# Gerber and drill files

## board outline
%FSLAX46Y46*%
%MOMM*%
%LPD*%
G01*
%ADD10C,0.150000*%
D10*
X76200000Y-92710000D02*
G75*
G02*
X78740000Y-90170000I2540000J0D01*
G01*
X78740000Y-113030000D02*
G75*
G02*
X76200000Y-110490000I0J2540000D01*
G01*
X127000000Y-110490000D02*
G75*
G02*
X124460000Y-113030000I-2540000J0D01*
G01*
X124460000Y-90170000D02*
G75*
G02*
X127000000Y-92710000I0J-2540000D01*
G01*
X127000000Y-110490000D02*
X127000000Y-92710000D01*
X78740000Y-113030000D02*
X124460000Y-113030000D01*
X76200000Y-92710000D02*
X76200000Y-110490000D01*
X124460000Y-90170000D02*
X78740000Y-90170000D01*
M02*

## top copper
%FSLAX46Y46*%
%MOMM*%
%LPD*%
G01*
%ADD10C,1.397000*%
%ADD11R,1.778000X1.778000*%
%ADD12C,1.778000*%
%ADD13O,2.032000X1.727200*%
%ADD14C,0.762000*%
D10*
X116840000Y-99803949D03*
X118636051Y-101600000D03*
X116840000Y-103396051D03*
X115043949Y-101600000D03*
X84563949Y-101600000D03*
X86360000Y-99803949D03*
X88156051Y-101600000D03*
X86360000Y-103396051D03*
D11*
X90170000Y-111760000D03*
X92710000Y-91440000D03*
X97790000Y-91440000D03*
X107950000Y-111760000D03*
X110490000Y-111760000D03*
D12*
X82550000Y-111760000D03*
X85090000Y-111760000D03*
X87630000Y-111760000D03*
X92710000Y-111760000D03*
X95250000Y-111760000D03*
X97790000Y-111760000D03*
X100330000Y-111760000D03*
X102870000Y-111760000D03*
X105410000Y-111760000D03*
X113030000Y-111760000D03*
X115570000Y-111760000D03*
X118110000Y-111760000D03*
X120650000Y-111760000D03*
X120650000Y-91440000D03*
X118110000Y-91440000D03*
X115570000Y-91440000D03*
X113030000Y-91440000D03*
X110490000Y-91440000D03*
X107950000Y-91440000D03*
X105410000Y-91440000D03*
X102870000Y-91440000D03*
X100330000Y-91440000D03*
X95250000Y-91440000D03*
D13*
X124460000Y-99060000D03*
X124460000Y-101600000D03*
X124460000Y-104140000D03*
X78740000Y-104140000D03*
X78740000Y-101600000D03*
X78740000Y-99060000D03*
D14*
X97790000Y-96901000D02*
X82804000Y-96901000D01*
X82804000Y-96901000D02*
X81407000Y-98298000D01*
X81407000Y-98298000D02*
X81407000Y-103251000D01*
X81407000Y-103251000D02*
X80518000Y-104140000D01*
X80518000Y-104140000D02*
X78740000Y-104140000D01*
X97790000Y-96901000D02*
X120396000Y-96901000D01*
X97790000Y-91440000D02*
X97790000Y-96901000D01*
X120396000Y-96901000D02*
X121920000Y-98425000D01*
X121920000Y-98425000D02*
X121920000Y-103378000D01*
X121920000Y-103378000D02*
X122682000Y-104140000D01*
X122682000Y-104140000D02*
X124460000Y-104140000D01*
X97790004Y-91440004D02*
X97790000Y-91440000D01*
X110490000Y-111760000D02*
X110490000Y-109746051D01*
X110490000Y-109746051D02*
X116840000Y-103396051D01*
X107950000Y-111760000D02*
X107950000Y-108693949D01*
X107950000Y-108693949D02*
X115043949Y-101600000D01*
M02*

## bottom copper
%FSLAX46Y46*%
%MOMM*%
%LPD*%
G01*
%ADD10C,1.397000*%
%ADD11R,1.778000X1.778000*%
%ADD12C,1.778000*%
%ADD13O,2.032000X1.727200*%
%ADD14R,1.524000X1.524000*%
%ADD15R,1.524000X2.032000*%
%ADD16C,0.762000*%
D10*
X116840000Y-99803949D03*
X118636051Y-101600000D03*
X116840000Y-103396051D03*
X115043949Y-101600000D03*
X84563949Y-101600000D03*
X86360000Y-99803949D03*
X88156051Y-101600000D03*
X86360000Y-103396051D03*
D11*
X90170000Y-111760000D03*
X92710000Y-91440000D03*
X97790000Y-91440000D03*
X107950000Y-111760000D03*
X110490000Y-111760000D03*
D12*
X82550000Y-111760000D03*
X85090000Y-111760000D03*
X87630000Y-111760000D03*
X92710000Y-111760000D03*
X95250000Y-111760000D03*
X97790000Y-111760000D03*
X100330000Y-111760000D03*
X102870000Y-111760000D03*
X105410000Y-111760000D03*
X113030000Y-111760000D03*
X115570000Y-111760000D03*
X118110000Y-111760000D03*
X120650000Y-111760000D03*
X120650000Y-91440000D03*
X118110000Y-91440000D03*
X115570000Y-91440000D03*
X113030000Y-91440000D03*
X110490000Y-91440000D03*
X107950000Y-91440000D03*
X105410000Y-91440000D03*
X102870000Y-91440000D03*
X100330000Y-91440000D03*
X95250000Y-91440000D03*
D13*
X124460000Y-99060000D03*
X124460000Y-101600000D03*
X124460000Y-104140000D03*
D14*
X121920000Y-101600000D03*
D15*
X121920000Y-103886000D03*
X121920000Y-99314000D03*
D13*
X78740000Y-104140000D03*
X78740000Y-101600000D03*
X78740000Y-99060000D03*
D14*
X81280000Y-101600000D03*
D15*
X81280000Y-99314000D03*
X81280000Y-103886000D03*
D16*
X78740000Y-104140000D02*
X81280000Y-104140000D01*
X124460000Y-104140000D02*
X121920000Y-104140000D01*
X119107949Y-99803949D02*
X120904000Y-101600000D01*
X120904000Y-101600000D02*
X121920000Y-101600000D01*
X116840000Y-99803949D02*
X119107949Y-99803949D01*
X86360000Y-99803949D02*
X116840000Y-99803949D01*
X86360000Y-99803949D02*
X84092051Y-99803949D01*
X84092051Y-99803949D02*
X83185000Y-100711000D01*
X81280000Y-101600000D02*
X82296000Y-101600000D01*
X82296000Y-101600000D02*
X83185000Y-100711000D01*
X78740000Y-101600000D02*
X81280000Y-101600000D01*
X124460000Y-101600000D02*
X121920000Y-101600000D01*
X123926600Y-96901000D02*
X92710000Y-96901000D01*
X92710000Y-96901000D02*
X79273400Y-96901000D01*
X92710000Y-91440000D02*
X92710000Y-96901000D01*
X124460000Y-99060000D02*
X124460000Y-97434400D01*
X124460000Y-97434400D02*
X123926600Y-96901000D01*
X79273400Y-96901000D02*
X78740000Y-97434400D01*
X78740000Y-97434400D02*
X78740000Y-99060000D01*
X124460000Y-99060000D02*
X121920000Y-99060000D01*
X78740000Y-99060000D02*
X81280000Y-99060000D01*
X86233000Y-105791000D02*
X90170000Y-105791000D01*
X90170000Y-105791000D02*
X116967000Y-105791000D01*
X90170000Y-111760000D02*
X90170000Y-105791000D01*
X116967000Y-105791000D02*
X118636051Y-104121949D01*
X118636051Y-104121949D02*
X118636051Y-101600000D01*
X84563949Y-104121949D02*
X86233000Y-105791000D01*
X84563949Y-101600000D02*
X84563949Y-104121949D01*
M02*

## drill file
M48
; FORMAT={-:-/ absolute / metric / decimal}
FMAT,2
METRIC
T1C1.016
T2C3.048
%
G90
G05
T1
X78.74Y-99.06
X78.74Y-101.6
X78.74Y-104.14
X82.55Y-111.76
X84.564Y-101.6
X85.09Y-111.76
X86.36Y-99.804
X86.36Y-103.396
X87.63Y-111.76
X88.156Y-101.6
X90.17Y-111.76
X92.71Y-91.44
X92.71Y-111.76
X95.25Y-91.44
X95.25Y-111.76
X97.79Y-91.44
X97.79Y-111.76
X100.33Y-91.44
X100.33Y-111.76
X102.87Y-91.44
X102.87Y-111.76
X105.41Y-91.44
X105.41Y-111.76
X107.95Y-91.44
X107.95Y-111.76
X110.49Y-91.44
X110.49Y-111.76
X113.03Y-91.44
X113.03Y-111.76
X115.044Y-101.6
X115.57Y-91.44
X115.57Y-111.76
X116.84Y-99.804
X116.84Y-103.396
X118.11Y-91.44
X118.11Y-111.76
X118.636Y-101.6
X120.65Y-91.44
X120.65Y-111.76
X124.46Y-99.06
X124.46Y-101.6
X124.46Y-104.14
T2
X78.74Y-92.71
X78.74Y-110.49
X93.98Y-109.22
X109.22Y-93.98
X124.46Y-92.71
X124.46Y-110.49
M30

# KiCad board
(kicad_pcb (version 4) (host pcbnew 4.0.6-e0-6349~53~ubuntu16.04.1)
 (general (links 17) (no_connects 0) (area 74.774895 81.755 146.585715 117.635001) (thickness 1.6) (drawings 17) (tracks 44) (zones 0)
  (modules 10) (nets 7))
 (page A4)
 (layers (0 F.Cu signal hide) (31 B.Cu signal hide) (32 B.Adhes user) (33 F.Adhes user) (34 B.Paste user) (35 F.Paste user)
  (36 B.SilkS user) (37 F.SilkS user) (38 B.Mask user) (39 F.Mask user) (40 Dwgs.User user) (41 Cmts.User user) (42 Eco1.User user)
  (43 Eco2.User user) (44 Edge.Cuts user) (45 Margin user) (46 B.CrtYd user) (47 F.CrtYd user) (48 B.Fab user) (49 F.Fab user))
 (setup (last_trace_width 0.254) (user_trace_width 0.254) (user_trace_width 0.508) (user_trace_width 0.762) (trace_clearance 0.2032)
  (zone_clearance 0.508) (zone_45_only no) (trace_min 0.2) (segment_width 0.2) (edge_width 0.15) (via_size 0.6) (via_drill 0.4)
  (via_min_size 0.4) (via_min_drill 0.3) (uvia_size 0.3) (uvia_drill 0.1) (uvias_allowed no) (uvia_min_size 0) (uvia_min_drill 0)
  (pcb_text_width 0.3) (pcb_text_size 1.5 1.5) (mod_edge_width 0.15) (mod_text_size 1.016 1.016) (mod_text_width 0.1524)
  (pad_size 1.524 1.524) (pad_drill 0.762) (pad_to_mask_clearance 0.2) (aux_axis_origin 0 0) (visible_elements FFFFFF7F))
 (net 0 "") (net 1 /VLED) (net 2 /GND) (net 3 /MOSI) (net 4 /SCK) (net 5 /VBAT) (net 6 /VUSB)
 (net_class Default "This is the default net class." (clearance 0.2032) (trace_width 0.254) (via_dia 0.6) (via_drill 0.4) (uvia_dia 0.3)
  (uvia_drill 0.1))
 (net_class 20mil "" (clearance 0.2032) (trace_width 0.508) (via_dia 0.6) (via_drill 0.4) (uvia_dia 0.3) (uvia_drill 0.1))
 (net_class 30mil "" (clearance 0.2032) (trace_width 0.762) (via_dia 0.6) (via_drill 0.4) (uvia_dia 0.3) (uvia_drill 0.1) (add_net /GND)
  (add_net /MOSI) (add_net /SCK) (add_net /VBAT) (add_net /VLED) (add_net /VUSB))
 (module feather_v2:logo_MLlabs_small (layer F.Cu) (at 107.95 101.6 90)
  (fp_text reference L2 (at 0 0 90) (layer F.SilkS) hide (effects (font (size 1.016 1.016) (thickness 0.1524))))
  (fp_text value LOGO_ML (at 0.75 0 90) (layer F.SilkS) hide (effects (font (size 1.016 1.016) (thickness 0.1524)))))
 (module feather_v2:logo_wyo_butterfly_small (layer F.Cu) (at 99.187 101.6 45)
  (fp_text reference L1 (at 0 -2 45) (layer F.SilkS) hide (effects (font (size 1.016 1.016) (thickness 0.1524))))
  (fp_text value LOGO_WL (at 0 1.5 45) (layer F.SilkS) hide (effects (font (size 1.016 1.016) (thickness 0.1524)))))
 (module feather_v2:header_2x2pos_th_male (layer B.Cu) (at 116.84 101.6 315)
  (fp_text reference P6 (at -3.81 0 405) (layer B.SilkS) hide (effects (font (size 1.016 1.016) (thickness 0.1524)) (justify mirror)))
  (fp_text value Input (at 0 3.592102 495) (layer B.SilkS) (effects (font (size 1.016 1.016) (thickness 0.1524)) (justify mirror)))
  (pad 1 thru_hole circle (at -1.27 -1.27 315) (size 1.397 1.397) (drill 1.016) (layers *.Cu *.Mask B.SilkS) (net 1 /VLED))
  (pad 3 thru_hole circle (at 1.27 -1.27 315) (size 1.397 1.397) (drill 1.016) (layers *.Cu *.Mask B.SilkS) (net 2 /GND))
  (pad 4 thru_hole circle (at 1.27 1.27 315) (size 1.397 1.397) (drill 1.016) (layers *.Cu *.Mask B.SilkS) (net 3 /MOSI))
  (pad 2 thru_hole circle (at -1.27 1.27 315) (size 1.397 1.397) (drill 1.016) (layers *.Cu *.Mask B.SilkS) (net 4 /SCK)))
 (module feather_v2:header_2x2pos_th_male (layer B.Cu) (at 86.36 101.6 45)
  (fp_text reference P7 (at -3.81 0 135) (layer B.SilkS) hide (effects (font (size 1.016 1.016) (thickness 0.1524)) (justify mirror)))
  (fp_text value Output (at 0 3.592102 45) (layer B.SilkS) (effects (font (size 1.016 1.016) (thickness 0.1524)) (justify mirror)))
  (pad 1 thru_hole circle (at -1.27 -1.27 45) (size 1.397 1.397) (drill 1.016) (layers *.Cu *.Mask B.SilkS) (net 2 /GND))
  (pad 3 thru_hole circle (at 1.27 -1.27 45) (size 1.397 1.397) (drill 1.016) (layers *.Cu *.Mask B.SilkS) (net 1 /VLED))
  (pad 4 thru_hole circle (at 1.27 1.27 45) (size 1.397 1.397) (drill 1.016) (layers *.Cu *.Mask B.SilkS))
  (pad 2 thru_hole circle (at -1.27 1.27 45) (size 1.397 1.397) (drill 1.016) (layers *.Cu *.Mask B.SilkS)))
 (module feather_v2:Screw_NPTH (layer F.Cu) (at 109.22 93.98)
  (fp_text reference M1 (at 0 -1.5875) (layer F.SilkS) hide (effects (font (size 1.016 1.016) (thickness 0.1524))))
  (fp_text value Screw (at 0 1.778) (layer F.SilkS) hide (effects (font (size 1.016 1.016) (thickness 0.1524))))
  (pad "" np_thru_hole circle (at 0 0) (size 3.048 3.048) (drill 3.048) (layers *.Cu *.Mask F.SilkS)))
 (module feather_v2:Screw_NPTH (layer F.Cu) (at 93.98 109.22)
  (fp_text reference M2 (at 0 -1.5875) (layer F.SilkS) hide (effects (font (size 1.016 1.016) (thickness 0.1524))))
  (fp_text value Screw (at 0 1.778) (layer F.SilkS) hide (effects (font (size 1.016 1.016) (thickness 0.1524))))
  (pad "" np_thru_hole circle (at 0 0) (size 3.048 3.048) (drill 3.048) (layers *.Cu *.Mask F.SilkS)))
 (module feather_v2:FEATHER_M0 (layer F.Cu) (at 101.6 101.6)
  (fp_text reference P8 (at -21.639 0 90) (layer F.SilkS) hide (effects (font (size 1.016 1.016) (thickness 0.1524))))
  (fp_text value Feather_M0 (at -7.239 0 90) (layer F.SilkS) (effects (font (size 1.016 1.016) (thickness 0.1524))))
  (pad 4 thru_hole rect (at -11.43 10.16) (size 1.778 1.778) (drill 1.016) (layers *.Cu *.Mask) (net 2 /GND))
  (pad 28 thru_hole rect (at -8.89 -10.16) (size 1.778 1.778) (drill 1.016) (layers *.Cu *.Mask) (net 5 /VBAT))
  (pad 26 thru_hole rect (at -3.81 -10.16) (size 1.778 1.778) (drill 1.016) (layers *.Cu *.Mask) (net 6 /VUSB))
  (pad 11 thru_hole rect (at 6.35 10.16) (size 1.778 1.778) (drill 1.016) (layers *.Cu *.Mask) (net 4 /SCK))
  (pad 12 thru_hole rect (at 8.89 10.16) (size 1.778 1.778) (drill 1.016) (layers *.Cu *.Mask) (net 3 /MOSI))
  (pad 1 thru_hole circle (at -19.05 10.16) (size 1.778 1.778) (drill 1.016) (layers *.Cu *.Mask))
  (pad 2 thru_hole circle (at -16.51 10.16) (size 1.778 1.778) (drill 1.016) (layers *.Cu *.Mask))
  (pad 3 thru_hole circle (at -13.97 10.16) (size 1.778 1.778) (drill 1.016) (layers *.Cu *.Mask))
  (pad 5 thru_hole circle (at -8.89 10.16) (size 1.778 1.778) (drill 1.016) (layers *.Cu *.Mask))
  (pad 6 thru_hole circle (at -6.35 10.16) (size 1.778 1.778) (drill 1.016) (layers *.Cu *.Mask))
  (pad 7 thru_hole circle (at -3.81 10.16) (size 1.778 1.778) (drill 1.016) (layers *.Cu *.Mask))
  (pad 8 thru_hole circle (at -1.27 10.16) (size 1.778 1.778) (drill 1.016) (layers *.Cu *.Mask))
  (pad 9 thru_hole circle (at 1.27 10.16) (size 1.778 1.778) (drill 1.016) (layers *.Cu *.Mask))
  (pad 10 thru_hole circle (at 3.81 10.16) (size 1.778 1.778) (drill 1.016) (layers *.Cu *.Mask))
  (pad 13 thru_hole circle (at 11.43 10.16) (size 1.778 1.778) (drill 1.016) (layers *.Cu *.Mask))
  (pad 14 thru_hole circle (at 13.97 10.16) (size 1.778 1.778) (drill 1.016) (layers *.Cu *.Mask))
  (pad 15 thru_hole circle (at 16.51 10.16) (size 1.778 1.778) (drill 1.016) (layers *.Cu *.Mask))
  (pad 16 thru_hole circle (at 19.05 10.16) (size 1.778 1.778) (drill 1.016) (layers *.Cu *.Mask))
  (pad 17 thru_hole circle (at 19.05 -10.16) (size 1.778 1.778) (drill 1.016) (layers *.Cu *.Mask))
  (pad 18 thru_hole circle (at 16.51 -10.16) (size 1.778 1.778) (drill 1.016) (layers *.Cu *.Mask))
  (pad 19 thru_hole circle (at 13.97 -10.16) (size 1.778 1.778) (drill 1.016) (layers *.Cu *.Mask))
  (pad 20 thru_hole circle (at 11.43 -10.16) (size 1.778 1.778) (drill 1.016) (layers *.Cu *.Mask))
  (pad 21 thru_hole circle (at 8.89 -10.16) (size 1.778 1.778) (drill 1.016) (layers *.Cu *.Mask))
  (pad 22 thru_hole circle (at 6.35 -10.16) (size 1.778 1.778) (drill 1.016) (layers *.Cu *.Mask))
  (pad 23 thru_hole circle (at 3.81 -10.16) (size 1.778 1.778) (drill 1.016) (layers *.Cu *.Mask))
  (pad 24 thru_hole circle (at 1.27 -10.16) (size 1.778 1.778) (drill 1.016) (layers *.Cu *.Mask))
  (pad 25 thru_hole circle (at -1.27 -10.16) (size 1.778 1.778) (drill 1.016) (layers *.Cu *.Mask))
  (pad 27 thru_hole circle (at -6.35 -10.16) (size 1.778 1.778) (drill 1.016) (layers *.Cu *.Mask))
  (pad "" np_thru_hole circle (at -22.86 8.89) (size 3.048 3.048) (drill 3.048) (layers *.Cu *.Mask))
  (pad "" np_thru_hole circle (at 22.86 8.89) (size 3.048 3.048) (drill 3.048) (layers *.Cu *.Mask))
  (pad "" np_thru_hole circle (at 22.86 -8.89) (size 3.048 3.048) (drill 3.048) (layers *.Cu *.Mask))
  (pad "" np_thru_hole circle (at -22.86 -8.89) (size 3.048 3.048) (drill 3.048) (layers *.Cu *.Mask)))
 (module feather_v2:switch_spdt (layer B.Cu) (at 124.46 101.6 180)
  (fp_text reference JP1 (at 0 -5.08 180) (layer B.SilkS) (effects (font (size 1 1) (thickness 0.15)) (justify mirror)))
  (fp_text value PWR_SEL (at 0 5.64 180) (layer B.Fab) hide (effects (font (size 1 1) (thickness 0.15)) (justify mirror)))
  (pad 1 thru_hole oval (at 0 2.54 180) (size 2.032 1.7272) (drill 1.016) (layers *.Cu *.Mask B.SilkS) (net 5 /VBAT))
  (pad 2 thru_hole oval (at 0 0 180) (size 2.032 1.7272) (drill 1.016) (layers *.Cu *.Mask B.SilkS) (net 1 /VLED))
  (pad 3 thru_hole oval (at 0 -2.54 180) (size 2.032 1.7272) (drill 1.016) (layers *.Cu *.Mask B.SilkS) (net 6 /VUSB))
  (pad 2 smd rect (at 2.54 0 180) (size 1.524 1.524) (layers B.Cu B.Paste B.Mask) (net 1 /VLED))
  (pad 3 smd rect (at 2.54 -2.54 180) (size 1.524 2.032) (drill (offset 0 0.254)) (layers B.Cu B.Paste B.Mask) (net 6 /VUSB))
  (pad 1 smd rect (at 2.54 2.54 180) (size 1.524 2.032) (drill (offset 0 -0.254)) (layers B.Cu B.Paste B.Mask) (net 5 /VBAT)))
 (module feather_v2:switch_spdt (layer B.Cu) (at 78.74 101.6)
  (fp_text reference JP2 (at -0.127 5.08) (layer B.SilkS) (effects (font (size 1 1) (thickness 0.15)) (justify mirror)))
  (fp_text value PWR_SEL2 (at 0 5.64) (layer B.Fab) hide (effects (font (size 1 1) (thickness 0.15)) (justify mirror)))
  (pad 1 thru_hole oval (at 0 2.54) (size 2.032 1.7272) (drill 1.016) (layers *.Cu *.Mask B.SilkS) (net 6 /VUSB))
  (pad 2 thru_hole oval (at 0 0) (size 2.032 1.7272) (drill 1.016) (layers *.Cu *.Mask B.SilkS) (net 1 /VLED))
  (pad 3 thru_hole oval (at 0 -2.54) (size 2.032 1.7272) (drill 1.016) (layers *.Cu *.Mask B.SilkS) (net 5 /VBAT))
  (pad 2 smd rect (at 2.54 0) (size 1.524 1.524) (layers B.Cu B.Paste B.Mask) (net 1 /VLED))
  (pad 3 smd rect (at 2.54 -2.54) (size 1.524 2.032) (drill (offset 0 0.254)) (layers B.Cu B.Paste B.Mask) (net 5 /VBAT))
  (pad 1 smd rect (at 2.54 2.54) (size 1.524 2.032) (drill (offset 0 -0.254)) (layers B.Cu B.Paste B.Mask) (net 6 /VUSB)))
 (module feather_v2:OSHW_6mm (layer B.Cu) (at 101.6 101.6 270)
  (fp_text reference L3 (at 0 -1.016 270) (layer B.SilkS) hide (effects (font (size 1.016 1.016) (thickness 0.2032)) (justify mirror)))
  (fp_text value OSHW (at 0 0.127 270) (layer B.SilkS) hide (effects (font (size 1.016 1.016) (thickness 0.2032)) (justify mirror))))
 (gr_arc (start 78.74 92.71) (end 76.2 92.71) (angle 90) (layer Edge.Cuts) (width 0.15))
 (gr_arc (start 78.74 110.49) (end 78.74 113.03) (angle 90) (layer Edge.Cuts) (width 0.15))
 (gr_arc (start 124.46 110.49) (end 127 110.49) (angle 90) (layer Edge.Cuts) (width 0.15))
 (gr_arc (start 124.46 92.71) (end 124.46 90.17) (angle 90) (layer Edge.Cuts) (width 0.15))
 (gr_line (start 127 110.49) (end 127 92.71) (layer Edge.Cuts) (width 0.15))
 (gr_line (start 78.74 113.03) (end 124.46 113.03) (layer Edge.Cuts) (width 0.15))
 (gr_line (start 76.2 92.71) (end 76.2 110.49) (layer Edge.Cuts) (width 0.15))
 (gr_line (start 124.46 90.17) (end 78.74 90.17) (layer Edge.Cuts) (width 0.15))
 (segment (start 97.79 96.901) (end 82.804 96.901) (width 0.762) (layer F.Cu) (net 6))
 (segment (start 82.804 96.901) (end 81.407 98.298) (width 0.762) (layer F.Cu) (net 6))
 (segment (start 81.407 98.298) (end 81.407 103.251) (width 0.762) (layer F.Cu) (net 6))
 (segment (start 81.407 103.251) (end 80.518 104.14) (width 0.762) (layer F.Cu) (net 6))
 (segment (start 80.518 104.14) (end 78.74 104.14) (width 0.762) (layer F.Cu) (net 6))
 (segment (start 97.79 96.901) (end 120.396 96.901) (width 0.762) (layer F.Cu) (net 6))
 (segment (start 97.79 91.44) (end 97.79 96.901) (width 0.762) (layer F.Cu) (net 6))
 (segment (start 120.396 96.901) (end 121.92 98.425) (width 0.762) (layer F.Cu) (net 6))
 (segment (start 121.92 98.425) (end 121.92 103.378) (width 0.762) (layer F.Cu) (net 6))
 (segment (start 121.92 103.378) (end 122.682 104.14) (width 0.762) (layer F.Cu) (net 6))
 (segment (start 122.682 104.14) (end 124.46 104.14) (width 0.762) (layer F.Cu) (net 6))
 (segment (start 78.74 104.14) (end 81.28 104.14) (width 0.762) (layer B.Cu) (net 6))
 (segment (start 97.790004 91.440004) (end 97.79 91.44) (width 0.762) (layer F.Cu) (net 6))
 (segment (start 124.46 104.14) (end 121.92 104.14) (width 0.762) (layer B.Cu) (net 6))
 (segment (start 119.107949 99.803949) (end 120.904 101.6) (width 0.762) (layer B.Cu) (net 1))
 (segment (start 120.904 101.6) (end 121.92 101.6) (width 0.762) (layer B.Cu) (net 1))
 (segment (start 116.84 99.803949) (end 119.107949 99.803949) (width 0.762) (layer B.Cu) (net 1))
 (segment (start 86.36 99.803949) (end 116.84 99.803949) (width 0.762) (layer B.Cu) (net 1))
 (segment (start 86.36 99.803949) (end 84.092051 99.803949) (width 0.762) (layer B.Cu) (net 1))
 (segment (start 84.092051 99.803949) (end 83.185 100.711) (width 0.762) (layer B.Cu) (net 1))
 (segment (start 81.28 101.6) (end 82.296 101.6) (width 0.762) (layer B.Cu) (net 1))
 (segment (start 82.296 101.6) (end 83.185 100.711) (width 0.762) (layer B.Cu) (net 1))
 (segment (start 78.74 101.6) (end 81.28 101.6) (width 0.762) (layer B.Cu) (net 1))
 (segment (start 124.46 101.6) (end 121.92 101.6) (width 0.762) (layer B.Cu) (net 1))
 (segment (start 123.9266 96.901) (end 92.71 96.901) (width 0.762) (layer B.Cu) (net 5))
 (segment (start 92.71 96.901) (end 79.2734 96.901) (width 0.762) (layer B.Cu) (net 5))
 (segment (start 92.71 91.44) (end 92.71 96.901) (width 0.762) (layer B.Cu) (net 5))
 (segment (start 124.46 99.06) (end 124.46 97.4344) (width 0.762) (layer B.Cu) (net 5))
 (segment (start 124.46 97.4344) (end 123.9266 96.901) (width 0.762) (layer B.Cu) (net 5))
 (segment (start 79.2734 96.901) (end 78.74 97.4344) (width 0.762) (layer B.Cu) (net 5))
 (segment (start 78.74 97.4344) (end 78.74 99.06) (width 0.762) (layer B.Cu) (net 5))
 (segment (start 124.46 99.06) (end 121.92 99.06) (width 0.762) (layer B.Cu) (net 5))
 (segment (start 78.74 99.06) (end 81.28 99.06) (width 0.762) (layer B.Cu) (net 5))
 (segment (start 86.233 105.791) (end 90.17 105.791) (width 0.762) (layer B.Cu) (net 2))
 (segment (start 90.17 105.791) (end 116.967 105.791) (width 0.762) (layer B.Cu) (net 2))
 (segment (start 90.17 111.76) (end 90.17 105.791) (width 0.762) (layer B.Cu) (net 2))
 (segment (start 116.967 105.791) (end 118.636051 104.121949) (width 0.762) (layer B.Cu) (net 2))
 (segment (start 118.636051 104.121949) (end 118.636051 101.6) (width 0.762) (layer B.Cu) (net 2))
 (segment (start 84.563949 104.121949) (end 86.233 105.791) (width 0.762) (layer B.Cu) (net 2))
 (segment (start 84.563949 101.6) (end 84.563949 104.121949) (width 0.762) (layer B.Cu) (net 2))
 (segment (start 110.49 111.76) (end 110.49 109.746051) (width 0.762) (layer F.Cu) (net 3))
 (segment (start 110.49 109.746051) (end 116.84 103.396051) (width 0.762) (layer F.Cu) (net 3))
 (segment (start 107.95 111.76) (end 107.95 108.693949) (width 0.762) (layer F.Cu) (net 4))
 (segment (start 107.95 108.693949) (end 115.043949 101.6) (width 0.762) (layer F.Cu) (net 4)))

